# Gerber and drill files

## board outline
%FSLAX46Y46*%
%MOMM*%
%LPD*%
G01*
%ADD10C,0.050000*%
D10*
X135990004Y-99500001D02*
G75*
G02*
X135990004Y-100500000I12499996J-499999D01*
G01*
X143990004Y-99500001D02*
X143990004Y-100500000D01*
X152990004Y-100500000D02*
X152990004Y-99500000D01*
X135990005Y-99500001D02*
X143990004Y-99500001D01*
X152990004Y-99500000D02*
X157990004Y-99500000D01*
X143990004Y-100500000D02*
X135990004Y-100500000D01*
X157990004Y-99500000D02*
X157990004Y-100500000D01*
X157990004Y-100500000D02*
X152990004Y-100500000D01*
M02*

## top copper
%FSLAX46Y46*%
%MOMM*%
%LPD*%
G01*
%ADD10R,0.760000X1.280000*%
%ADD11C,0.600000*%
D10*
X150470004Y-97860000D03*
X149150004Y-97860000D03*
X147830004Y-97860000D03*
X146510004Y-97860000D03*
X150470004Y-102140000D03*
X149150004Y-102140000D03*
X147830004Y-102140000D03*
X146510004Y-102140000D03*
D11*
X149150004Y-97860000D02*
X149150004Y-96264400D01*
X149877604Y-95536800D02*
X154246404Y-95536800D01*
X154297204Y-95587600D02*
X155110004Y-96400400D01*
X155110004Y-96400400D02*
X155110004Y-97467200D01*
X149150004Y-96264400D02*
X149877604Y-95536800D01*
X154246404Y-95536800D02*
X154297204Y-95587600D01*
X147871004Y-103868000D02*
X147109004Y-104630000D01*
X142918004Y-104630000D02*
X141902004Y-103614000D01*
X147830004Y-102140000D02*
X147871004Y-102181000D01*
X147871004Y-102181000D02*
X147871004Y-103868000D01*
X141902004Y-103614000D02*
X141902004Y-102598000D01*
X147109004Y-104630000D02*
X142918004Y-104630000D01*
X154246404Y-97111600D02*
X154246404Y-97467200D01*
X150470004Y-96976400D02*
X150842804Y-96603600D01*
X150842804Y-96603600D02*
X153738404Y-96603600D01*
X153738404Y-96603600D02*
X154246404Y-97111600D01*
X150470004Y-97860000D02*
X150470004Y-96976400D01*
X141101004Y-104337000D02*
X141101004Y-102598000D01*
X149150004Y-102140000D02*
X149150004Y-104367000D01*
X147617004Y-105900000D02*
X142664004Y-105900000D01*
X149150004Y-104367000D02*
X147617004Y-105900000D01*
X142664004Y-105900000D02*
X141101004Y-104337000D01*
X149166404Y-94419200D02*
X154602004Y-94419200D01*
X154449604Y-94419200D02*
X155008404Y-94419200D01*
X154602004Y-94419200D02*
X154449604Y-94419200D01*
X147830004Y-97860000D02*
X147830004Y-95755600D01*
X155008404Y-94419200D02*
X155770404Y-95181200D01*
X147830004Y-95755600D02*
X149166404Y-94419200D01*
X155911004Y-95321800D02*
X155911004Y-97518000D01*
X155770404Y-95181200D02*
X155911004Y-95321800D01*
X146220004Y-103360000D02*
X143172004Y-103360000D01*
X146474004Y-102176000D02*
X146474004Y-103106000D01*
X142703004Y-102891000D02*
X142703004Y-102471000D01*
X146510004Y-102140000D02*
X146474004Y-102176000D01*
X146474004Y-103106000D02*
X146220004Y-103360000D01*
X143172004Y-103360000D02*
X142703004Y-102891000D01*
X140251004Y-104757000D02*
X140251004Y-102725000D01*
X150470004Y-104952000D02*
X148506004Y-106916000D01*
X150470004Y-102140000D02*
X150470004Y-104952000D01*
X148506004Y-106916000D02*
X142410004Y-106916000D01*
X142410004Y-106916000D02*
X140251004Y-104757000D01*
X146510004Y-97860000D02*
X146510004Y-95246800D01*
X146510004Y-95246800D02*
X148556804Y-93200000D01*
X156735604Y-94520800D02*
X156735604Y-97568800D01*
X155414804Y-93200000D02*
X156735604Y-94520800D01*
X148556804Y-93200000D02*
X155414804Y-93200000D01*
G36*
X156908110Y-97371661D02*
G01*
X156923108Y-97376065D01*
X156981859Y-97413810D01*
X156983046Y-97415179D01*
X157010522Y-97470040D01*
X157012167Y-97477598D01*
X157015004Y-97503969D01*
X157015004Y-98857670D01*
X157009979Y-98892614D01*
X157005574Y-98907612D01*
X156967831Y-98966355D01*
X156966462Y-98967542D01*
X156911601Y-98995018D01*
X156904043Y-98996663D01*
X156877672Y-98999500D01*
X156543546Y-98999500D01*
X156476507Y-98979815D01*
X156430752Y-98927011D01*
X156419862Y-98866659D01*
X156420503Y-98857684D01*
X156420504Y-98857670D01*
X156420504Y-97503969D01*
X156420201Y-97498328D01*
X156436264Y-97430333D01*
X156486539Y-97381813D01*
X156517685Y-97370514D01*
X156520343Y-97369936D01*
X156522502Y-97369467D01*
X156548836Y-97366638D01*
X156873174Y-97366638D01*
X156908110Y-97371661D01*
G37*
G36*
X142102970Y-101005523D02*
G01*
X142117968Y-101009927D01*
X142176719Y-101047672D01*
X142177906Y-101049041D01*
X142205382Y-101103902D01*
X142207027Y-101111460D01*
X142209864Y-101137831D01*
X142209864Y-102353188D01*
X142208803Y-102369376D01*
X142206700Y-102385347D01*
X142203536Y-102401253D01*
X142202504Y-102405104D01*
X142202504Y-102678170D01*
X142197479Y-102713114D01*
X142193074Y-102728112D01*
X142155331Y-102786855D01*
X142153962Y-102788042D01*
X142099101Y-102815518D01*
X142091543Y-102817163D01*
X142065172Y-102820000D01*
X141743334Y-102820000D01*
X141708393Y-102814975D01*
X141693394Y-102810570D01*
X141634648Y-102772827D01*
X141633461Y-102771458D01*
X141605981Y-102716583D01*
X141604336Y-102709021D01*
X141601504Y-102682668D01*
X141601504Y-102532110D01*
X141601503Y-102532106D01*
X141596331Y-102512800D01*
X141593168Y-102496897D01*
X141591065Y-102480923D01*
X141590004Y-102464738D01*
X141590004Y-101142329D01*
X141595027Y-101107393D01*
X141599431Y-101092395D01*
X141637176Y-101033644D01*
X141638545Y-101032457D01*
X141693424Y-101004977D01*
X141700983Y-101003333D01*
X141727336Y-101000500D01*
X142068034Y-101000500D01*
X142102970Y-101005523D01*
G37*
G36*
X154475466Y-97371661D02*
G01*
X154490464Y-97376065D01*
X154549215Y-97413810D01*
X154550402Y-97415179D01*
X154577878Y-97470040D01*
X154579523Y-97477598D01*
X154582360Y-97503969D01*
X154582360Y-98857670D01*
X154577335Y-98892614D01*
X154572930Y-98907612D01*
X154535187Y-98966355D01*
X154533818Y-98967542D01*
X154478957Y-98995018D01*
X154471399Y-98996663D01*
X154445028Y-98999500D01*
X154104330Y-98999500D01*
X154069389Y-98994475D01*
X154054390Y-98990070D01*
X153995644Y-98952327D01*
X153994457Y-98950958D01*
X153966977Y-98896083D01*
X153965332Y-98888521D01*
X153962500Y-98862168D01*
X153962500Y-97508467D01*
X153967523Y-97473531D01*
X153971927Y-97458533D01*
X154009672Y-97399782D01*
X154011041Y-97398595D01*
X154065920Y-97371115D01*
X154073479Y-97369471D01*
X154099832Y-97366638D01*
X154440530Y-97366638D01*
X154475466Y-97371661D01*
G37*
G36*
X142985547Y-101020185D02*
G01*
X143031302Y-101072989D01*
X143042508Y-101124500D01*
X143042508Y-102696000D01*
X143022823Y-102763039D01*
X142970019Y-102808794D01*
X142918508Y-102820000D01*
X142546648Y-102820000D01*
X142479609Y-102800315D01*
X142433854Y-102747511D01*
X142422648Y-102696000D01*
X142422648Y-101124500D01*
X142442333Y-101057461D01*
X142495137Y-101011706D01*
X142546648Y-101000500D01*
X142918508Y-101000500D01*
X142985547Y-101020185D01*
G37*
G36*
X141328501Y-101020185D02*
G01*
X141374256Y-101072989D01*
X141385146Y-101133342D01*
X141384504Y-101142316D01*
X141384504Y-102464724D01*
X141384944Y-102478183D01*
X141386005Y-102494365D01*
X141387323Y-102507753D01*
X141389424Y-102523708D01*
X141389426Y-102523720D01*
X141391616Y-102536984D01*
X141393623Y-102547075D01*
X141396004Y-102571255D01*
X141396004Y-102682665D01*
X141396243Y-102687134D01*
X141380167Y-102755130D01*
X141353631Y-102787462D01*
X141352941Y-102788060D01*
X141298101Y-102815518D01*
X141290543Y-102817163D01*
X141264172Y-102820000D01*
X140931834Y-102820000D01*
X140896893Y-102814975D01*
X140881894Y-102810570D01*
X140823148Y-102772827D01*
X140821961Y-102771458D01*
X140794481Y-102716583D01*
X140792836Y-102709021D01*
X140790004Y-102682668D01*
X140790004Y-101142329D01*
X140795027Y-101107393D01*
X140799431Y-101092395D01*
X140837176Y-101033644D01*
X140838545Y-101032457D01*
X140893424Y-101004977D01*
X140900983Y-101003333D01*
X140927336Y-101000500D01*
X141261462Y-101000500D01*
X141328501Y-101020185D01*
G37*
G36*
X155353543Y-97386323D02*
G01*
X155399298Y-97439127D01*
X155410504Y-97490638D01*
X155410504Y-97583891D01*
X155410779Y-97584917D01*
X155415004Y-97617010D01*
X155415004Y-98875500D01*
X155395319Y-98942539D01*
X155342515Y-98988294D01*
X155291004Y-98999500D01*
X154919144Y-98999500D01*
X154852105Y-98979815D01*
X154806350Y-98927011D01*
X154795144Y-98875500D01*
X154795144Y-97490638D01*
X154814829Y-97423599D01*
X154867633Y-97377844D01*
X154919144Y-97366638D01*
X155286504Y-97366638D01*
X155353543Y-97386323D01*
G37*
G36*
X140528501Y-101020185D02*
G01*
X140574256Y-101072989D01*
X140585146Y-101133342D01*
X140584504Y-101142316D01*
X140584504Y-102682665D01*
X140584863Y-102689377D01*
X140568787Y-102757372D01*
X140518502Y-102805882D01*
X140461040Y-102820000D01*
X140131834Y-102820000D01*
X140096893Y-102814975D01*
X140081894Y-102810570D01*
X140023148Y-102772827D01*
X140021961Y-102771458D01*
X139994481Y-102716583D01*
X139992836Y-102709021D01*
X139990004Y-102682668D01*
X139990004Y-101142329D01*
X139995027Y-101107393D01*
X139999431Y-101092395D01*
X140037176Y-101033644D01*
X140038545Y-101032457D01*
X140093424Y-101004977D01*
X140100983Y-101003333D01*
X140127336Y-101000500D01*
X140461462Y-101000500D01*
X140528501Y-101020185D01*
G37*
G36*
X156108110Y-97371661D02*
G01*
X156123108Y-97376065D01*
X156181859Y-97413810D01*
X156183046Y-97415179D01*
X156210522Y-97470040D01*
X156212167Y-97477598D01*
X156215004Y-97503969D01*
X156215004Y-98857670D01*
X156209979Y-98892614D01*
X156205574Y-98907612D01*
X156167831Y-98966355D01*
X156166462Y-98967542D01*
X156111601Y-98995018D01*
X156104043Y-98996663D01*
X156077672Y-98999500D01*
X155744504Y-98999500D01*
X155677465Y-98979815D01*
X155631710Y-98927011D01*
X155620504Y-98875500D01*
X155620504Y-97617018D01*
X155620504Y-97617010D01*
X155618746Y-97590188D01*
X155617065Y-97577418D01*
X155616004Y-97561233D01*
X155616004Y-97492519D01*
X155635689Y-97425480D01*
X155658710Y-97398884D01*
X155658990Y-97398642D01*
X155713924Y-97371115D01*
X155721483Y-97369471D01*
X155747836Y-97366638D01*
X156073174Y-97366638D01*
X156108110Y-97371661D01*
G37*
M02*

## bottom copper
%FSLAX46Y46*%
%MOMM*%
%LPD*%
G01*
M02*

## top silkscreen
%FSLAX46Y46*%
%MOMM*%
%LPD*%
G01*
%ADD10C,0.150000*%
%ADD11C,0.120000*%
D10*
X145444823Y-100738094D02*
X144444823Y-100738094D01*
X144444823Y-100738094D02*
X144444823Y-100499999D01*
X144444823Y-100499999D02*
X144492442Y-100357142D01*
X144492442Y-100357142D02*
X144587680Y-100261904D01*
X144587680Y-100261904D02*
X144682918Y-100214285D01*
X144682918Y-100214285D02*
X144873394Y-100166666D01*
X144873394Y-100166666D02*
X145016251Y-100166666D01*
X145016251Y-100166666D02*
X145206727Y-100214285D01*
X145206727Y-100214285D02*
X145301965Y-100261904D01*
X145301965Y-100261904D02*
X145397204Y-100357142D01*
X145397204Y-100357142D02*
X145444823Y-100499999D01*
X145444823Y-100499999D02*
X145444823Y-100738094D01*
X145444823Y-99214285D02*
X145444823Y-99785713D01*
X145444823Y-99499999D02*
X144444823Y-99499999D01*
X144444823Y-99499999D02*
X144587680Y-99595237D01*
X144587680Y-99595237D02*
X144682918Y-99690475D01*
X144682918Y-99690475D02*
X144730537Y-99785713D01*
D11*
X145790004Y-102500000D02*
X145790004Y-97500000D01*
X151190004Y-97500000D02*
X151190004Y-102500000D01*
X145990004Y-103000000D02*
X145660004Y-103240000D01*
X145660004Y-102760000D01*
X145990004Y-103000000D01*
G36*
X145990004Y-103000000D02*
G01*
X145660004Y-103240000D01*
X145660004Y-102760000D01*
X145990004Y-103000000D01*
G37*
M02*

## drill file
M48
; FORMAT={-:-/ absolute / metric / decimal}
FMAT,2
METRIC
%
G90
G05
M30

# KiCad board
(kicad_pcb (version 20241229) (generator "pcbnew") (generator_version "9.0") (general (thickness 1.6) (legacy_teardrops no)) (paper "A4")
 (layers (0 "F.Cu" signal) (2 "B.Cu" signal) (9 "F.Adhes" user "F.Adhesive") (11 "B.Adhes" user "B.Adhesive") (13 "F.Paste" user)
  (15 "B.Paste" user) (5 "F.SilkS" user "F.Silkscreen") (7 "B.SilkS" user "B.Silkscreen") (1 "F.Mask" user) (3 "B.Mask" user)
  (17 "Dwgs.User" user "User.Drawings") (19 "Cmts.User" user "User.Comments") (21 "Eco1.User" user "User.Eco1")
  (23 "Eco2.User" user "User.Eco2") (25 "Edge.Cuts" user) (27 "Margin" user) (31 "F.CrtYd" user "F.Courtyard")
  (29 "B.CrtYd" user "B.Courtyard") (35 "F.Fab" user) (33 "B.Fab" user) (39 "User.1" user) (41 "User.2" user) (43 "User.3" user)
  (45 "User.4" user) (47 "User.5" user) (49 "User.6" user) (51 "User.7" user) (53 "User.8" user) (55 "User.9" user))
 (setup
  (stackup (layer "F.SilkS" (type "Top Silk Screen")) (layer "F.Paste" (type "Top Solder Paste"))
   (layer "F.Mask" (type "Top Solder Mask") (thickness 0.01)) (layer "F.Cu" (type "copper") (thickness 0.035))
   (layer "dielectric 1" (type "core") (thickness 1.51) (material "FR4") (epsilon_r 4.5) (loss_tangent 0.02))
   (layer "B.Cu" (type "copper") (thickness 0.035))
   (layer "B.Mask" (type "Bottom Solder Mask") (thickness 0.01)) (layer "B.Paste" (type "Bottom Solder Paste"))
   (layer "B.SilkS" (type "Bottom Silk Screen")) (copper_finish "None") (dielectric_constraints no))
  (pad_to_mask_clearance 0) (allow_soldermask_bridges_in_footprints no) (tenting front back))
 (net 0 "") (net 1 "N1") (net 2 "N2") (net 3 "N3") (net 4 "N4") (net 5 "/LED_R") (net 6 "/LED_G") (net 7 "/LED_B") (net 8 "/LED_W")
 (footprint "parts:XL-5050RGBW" (layer "F.Cu") (at 148.490004 100 -90)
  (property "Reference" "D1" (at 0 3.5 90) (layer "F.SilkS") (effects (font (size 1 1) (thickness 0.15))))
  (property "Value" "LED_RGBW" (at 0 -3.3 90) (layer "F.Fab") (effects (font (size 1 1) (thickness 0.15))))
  (fp_line (start 2.5 2.7) (end -2.5 2.7) (stroke (width 0.12) (type solid)) (layer "F.SilkS"))
  (fp_line (start -2.5 -2.7) (end 2.5 -2.7) (stroke (width 0.12) (type solid)) (layer "F.SilkS"))
  (fp_poly (pts (xy 3 2.5) (xy 3.24 2.83) (xy 2.76 2.83) (xy 3 2.5)) (stroke (width 0.12) (type solid)) (fill yes) (layer "F.SilkS"))
  (pad "1" smd rect (at -2.14 -1.98) (size 0.76 1.28) (layers "F.Cu" "F.Mask" "F.Paste") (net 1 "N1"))
  (pad "2" smd rect (at -2.14 -0.66) (size 0.76 1.28) (layers "F.Cu" "F.Mask" "F.Paste") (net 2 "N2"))
  (pad "3" smd rect (at -2.14 0.66) (size 0.76 1.28) (layers "F.Cu" "F.Mask" "F.Paste") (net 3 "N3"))
  (pad "4" smd rect (at -2.14 1.98) (size 0.76 1.28) (layers "F.Cu" "F.Mask" "F.Paste") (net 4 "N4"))
  (pad "5" smd rect (at 2.14 -1.98) (size 0.76 1.28) (layers "F.Cu" "F.Mask" "F.Paste") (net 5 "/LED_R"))
  (pad "6" smd rect (at 2.14 -0.66) (size 0.76 1.28) (layers "F.Cu" "F.Mask" "F.Paste") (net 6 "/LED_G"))
  (pad "7" smd rect (at 2.14 0.66) (size 0.76 1.28) (layers "F.Cu" "F.Mask" "F.Paste") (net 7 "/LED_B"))
  (pad "8" smd rect (at 2.14 1.98) (size 0.76 1.28) (layers "F.Cu" "F.Mask" "F.Paste") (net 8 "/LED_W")))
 (gr_arc (start 135.990004 99.500001) (mid 161 100) (end 135.990004 100.5) (stroke (width 0.05) (type default)) (layer "Edge.Cuts"))
 (gr_line (start 143.990004 99.500001) (end 143.990004 100.5) (stroke (width 0.05) (type default)) (layer "Edge.Cuts"))
 (gr_line (start 152.990004 100.5) (end 152.990004 99.5) (stroke (width 0.05) (type default)) (layer "Edge.Cuts"))
 (gr_line (start 135.990005 99.500001) (end 143.990004 99.500001) (stroke (width 0.05) (type default)) (layer "Edge.Cuts"))
 (gr_line (start 152.990004 99.5) (end 157.990004 99.5) (stroke (width 0.05) (type default)) (layer "Edge.Cuts"))
 (gr_line (start 143.990004 100.5) (end 135.990004 100.5) (stroke (width 0.05) (type default)) (layer "Edge.Cuts"))
 (gr_line (start 157.990004 99.5) (end 157.990004 100.5) (stroke (width 0.05) (type default)) (layer "Edge.Cuts"))
 (gr_line (start 157.990004 100.5) (end 152.990004 100.5) (stroke (width 0.05) (type default)) (layer "Edge.Cuts"))
 (segment (start 149.150004 97.86) (end 149.150004 96.2644) (width 0.6) (layer "F.Cu") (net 2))
 (segment (start 149.877604 95.5368) (end 154.246404 95.5368) (width 0.6) (layer "F.Cu") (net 2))
 (segment (start 154.297204 95.5876) (end 155.110004 96.4004) (width 0.6) (layer "F.Cu") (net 2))
 (segment (start 155.110004 96.4004) (end 155.110004 97.4672) (width 0.6) (layer "F.Cu") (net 2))
 (segment (start 149.150004 96.2644) (end 149.877604 95.5368) (width 0.6) (layer "F.Cu") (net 2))
 (segment (start 154.246404 95.5368) (end 154.297204 95.5876) (width 0.6) (layer "F.Cu") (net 2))
 (segment (start 147.871004 103.868) (end 147.109004 104.63) (width 0.6) (layer "F.Cu") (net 7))
 (segment (start 142.918004 104.63) (end 141.902004 103.614) (width 0.6) (layer "F.Cu") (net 7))
 (segment (start 147.830004 102.14) (end 147.871004 102.181) (width 0.6) (layer "F.Cu") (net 7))
 (segment (start 147.871004 102.181) (end 147.871004 103.868) (width 0.6) (layer "F.Cu") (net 7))
 (segment (start 141.902004 103.614) (end 141.902004 102.598) (width 0.6) (layer "F.Cu") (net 7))
 (segment (start 147.109004 104.63) (end 142.918004 104.63) (width 0.6) (layer "F.Cu") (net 7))
 (segment (start 154.246404 97.1116) (end 154.246404 97.4672) (width 0.6) (layer "F.Cu") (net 1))
 (segment (start 150.470004 96.9764) (end 150.842804 96.6036) (width 0.6) (layer "F.Cu") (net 1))
 (segment (start 150.842804 96.6036) (end 153.738404 96.6036) (width 0.6) (layer "F.Cu") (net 1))
 (segment (start 153.738404 96.6036) (end 154.246404 97.1116) (width 0.6) (layer "F.Cu") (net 1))
 (segment (start 150.470004 97.86) (end 150.470004 96.9764) (width 0.6) (layer "F.Cu") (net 1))
 (segment (start 141.101004 104.337) (end 141.101004 102.598) (width 0.6) (layer "F.Cu") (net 6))
 (segment (start 149.150004 102.14) (end 149.150004 104.367) (width 0.6) (layer "F.Cu") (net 6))
 (segment (start 147.617004 105.9) (end 142.664004 105.9) (width 0.6) (layer "F.Cu") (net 6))
 (segment (start 149.150004 104.367) (end 147.617004 105.9) (width 0.6) (layer "F.Cu") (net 6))
 (segment (start 142.664004 105.9) (end 141.101004 104.337) (width 0.6) (layer "F.Cu") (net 6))
 (segment (start 149.166404 94.4192) (end 154.602004 94.4192) (width 0.6) (layer "F.Cu") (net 3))
 (segment (start 154.449604 94.4192) (end 155.008404 94.4192) (width 0.6) (layer "F.Cu") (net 3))
 (segment (start 154.602004 94.4192) (end 154.449604 94.4192) (width 0.6) (layer "F.Cu") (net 3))
 (segment (start 147.830004 97.86) (end 147.830004 95.7556) (width 0.6) (layer "F.Cu") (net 3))
 (segment (start 155.008404 94.4192) (end 155.770404 95.1812) (width 0.6) (layer "F.Cu") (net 3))
 (segment (start 147.830004 95.7556) (end 149.166404 94.4192) (width 0.6) (layer "F.Cu") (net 3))
 (segment (start 155.911004 95.3218) (end 155.911004 97.518) (width 0.6) (layer "F.Cu") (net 3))
 (segment (start 155.770404 95.1812) (end 155.911004 95.3218) (width 0.6) (layer "F.Cu") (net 3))
 (segment (start 146.220004 103.36) (end 143.172004 103.36) (width 0.6) (layer "F.Cu") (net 8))
 (segment (start 146.474004 102.176) (end 146.474004 103.106) (width 0.6) (layer "F.Cu") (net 8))
 (segment (start 142.703004 102.891) (end 142.703004 102.471) (width 0.6) (layer "F.Cu") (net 8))
 (segment (start 146.510004 102.14) (end 146.474004 102.176) (width 0.6) (layer "F.Cu") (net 8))
 (segment (start 146.474004 103.106) (end 146.220004 103.36) (width 0.6) (layer "F.Cu") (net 8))
 (segment (start 143.172004 103.36) (end 142.703004 102.891) (width 0.6) (layer "F.Cu") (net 8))
 (segment (start 140.251004 104.757) (end 140.251004 102.725) (width 0.6) (layer "F.Cu") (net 5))
 (segment (start 150.470004 104.952) (end 148.506004 106.916) (width 0.6) (layer "F.Cu") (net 5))
 (segment (start 150.470004 102.14) (end 150.470004 104.952) (width 0.6) (layer "F.Cu") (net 5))
 (segment (start 148.506004 106.916) (end 142.410004 106.916) (width 0.6) (layer "F.Cu") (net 5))
 (segment (start 142.410004 106.916) (end 140.251004 104.757) (width 0.6) (layer "F.Cu") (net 5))
 (segment (start 146.510004 97.86) (end 146.510004 95.2468) (width 0.6) (layer "F.Cu") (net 4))
 (segment (start 146.510004 95.2468) (end 148.556804 93.2) (width 0.6) (layer "F.Cu") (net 4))
 (segment (start 156.735604 94.5208) (end 156.735604 97.5688) (width 0.6) (layer "F.Cu") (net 4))
 (segment (start 155.414804 93.2) (end 156.735604 94.5208) (width 0.6) (layer "F.Cu") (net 4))
 (segment (start 148.556804 93.2) (end 155.414804 93.2) (width 0.6) (layer "F.Cu") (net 4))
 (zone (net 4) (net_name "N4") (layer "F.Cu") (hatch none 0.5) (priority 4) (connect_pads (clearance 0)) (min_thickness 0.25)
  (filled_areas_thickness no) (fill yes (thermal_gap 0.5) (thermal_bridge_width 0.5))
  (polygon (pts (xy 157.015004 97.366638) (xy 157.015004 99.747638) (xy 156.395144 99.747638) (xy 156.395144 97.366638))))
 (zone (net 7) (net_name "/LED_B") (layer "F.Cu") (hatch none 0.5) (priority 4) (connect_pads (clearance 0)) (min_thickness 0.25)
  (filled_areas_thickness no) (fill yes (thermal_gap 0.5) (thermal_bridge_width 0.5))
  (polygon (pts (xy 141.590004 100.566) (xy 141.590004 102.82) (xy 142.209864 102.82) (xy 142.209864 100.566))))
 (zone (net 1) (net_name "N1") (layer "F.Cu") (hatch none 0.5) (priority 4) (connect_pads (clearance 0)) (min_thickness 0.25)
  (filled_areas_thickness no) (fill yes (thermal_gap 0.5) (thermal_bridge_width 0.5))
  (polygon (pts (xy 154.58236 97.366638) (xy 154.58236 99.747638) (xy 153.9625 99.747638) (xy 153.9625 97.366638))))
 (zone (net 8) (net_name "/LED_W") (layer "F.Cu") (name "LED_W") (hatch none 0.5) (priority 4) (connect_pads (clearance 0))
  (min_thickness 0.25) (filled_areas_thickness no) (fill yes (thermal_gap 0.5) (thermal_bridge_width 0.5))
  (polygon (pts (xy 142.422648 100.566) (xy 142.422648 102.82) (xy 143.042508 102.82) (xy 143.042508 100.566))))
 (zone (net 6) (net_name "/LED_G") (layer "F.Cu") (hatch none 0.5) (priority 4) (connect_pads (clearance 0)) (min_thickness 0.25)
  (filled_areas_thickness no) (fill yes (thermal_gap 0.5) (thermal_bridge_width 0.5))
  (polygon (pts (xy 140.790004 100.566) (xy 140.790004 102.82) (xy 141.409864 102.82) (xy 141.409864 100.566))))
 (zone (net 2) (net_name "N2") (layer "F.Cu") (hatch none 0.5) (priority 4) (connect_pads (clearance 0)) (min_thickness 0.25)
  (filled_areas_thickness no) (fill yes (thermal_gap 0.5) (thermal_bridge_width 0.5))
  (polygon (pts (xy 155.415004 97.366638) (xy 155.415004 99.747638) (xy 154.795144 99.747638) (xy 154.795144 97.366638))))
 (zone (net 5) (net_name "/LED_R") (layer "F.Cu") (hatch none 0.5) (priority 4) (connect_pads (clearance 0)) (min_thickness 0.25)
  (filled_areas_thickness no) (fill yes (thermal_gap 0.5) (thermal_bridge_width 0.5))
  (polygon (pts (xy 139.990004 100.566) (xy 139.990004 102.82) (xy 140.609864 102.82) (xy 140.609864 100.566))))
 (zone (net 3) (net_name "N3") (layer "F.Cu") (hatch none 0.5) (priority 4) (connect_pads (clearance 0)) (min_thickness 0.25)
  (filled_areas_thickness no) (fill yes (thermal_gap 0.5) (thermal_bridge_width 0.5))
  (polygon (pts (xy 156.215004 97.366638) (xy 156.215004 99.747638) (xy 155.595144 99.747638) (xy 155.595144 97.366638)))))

